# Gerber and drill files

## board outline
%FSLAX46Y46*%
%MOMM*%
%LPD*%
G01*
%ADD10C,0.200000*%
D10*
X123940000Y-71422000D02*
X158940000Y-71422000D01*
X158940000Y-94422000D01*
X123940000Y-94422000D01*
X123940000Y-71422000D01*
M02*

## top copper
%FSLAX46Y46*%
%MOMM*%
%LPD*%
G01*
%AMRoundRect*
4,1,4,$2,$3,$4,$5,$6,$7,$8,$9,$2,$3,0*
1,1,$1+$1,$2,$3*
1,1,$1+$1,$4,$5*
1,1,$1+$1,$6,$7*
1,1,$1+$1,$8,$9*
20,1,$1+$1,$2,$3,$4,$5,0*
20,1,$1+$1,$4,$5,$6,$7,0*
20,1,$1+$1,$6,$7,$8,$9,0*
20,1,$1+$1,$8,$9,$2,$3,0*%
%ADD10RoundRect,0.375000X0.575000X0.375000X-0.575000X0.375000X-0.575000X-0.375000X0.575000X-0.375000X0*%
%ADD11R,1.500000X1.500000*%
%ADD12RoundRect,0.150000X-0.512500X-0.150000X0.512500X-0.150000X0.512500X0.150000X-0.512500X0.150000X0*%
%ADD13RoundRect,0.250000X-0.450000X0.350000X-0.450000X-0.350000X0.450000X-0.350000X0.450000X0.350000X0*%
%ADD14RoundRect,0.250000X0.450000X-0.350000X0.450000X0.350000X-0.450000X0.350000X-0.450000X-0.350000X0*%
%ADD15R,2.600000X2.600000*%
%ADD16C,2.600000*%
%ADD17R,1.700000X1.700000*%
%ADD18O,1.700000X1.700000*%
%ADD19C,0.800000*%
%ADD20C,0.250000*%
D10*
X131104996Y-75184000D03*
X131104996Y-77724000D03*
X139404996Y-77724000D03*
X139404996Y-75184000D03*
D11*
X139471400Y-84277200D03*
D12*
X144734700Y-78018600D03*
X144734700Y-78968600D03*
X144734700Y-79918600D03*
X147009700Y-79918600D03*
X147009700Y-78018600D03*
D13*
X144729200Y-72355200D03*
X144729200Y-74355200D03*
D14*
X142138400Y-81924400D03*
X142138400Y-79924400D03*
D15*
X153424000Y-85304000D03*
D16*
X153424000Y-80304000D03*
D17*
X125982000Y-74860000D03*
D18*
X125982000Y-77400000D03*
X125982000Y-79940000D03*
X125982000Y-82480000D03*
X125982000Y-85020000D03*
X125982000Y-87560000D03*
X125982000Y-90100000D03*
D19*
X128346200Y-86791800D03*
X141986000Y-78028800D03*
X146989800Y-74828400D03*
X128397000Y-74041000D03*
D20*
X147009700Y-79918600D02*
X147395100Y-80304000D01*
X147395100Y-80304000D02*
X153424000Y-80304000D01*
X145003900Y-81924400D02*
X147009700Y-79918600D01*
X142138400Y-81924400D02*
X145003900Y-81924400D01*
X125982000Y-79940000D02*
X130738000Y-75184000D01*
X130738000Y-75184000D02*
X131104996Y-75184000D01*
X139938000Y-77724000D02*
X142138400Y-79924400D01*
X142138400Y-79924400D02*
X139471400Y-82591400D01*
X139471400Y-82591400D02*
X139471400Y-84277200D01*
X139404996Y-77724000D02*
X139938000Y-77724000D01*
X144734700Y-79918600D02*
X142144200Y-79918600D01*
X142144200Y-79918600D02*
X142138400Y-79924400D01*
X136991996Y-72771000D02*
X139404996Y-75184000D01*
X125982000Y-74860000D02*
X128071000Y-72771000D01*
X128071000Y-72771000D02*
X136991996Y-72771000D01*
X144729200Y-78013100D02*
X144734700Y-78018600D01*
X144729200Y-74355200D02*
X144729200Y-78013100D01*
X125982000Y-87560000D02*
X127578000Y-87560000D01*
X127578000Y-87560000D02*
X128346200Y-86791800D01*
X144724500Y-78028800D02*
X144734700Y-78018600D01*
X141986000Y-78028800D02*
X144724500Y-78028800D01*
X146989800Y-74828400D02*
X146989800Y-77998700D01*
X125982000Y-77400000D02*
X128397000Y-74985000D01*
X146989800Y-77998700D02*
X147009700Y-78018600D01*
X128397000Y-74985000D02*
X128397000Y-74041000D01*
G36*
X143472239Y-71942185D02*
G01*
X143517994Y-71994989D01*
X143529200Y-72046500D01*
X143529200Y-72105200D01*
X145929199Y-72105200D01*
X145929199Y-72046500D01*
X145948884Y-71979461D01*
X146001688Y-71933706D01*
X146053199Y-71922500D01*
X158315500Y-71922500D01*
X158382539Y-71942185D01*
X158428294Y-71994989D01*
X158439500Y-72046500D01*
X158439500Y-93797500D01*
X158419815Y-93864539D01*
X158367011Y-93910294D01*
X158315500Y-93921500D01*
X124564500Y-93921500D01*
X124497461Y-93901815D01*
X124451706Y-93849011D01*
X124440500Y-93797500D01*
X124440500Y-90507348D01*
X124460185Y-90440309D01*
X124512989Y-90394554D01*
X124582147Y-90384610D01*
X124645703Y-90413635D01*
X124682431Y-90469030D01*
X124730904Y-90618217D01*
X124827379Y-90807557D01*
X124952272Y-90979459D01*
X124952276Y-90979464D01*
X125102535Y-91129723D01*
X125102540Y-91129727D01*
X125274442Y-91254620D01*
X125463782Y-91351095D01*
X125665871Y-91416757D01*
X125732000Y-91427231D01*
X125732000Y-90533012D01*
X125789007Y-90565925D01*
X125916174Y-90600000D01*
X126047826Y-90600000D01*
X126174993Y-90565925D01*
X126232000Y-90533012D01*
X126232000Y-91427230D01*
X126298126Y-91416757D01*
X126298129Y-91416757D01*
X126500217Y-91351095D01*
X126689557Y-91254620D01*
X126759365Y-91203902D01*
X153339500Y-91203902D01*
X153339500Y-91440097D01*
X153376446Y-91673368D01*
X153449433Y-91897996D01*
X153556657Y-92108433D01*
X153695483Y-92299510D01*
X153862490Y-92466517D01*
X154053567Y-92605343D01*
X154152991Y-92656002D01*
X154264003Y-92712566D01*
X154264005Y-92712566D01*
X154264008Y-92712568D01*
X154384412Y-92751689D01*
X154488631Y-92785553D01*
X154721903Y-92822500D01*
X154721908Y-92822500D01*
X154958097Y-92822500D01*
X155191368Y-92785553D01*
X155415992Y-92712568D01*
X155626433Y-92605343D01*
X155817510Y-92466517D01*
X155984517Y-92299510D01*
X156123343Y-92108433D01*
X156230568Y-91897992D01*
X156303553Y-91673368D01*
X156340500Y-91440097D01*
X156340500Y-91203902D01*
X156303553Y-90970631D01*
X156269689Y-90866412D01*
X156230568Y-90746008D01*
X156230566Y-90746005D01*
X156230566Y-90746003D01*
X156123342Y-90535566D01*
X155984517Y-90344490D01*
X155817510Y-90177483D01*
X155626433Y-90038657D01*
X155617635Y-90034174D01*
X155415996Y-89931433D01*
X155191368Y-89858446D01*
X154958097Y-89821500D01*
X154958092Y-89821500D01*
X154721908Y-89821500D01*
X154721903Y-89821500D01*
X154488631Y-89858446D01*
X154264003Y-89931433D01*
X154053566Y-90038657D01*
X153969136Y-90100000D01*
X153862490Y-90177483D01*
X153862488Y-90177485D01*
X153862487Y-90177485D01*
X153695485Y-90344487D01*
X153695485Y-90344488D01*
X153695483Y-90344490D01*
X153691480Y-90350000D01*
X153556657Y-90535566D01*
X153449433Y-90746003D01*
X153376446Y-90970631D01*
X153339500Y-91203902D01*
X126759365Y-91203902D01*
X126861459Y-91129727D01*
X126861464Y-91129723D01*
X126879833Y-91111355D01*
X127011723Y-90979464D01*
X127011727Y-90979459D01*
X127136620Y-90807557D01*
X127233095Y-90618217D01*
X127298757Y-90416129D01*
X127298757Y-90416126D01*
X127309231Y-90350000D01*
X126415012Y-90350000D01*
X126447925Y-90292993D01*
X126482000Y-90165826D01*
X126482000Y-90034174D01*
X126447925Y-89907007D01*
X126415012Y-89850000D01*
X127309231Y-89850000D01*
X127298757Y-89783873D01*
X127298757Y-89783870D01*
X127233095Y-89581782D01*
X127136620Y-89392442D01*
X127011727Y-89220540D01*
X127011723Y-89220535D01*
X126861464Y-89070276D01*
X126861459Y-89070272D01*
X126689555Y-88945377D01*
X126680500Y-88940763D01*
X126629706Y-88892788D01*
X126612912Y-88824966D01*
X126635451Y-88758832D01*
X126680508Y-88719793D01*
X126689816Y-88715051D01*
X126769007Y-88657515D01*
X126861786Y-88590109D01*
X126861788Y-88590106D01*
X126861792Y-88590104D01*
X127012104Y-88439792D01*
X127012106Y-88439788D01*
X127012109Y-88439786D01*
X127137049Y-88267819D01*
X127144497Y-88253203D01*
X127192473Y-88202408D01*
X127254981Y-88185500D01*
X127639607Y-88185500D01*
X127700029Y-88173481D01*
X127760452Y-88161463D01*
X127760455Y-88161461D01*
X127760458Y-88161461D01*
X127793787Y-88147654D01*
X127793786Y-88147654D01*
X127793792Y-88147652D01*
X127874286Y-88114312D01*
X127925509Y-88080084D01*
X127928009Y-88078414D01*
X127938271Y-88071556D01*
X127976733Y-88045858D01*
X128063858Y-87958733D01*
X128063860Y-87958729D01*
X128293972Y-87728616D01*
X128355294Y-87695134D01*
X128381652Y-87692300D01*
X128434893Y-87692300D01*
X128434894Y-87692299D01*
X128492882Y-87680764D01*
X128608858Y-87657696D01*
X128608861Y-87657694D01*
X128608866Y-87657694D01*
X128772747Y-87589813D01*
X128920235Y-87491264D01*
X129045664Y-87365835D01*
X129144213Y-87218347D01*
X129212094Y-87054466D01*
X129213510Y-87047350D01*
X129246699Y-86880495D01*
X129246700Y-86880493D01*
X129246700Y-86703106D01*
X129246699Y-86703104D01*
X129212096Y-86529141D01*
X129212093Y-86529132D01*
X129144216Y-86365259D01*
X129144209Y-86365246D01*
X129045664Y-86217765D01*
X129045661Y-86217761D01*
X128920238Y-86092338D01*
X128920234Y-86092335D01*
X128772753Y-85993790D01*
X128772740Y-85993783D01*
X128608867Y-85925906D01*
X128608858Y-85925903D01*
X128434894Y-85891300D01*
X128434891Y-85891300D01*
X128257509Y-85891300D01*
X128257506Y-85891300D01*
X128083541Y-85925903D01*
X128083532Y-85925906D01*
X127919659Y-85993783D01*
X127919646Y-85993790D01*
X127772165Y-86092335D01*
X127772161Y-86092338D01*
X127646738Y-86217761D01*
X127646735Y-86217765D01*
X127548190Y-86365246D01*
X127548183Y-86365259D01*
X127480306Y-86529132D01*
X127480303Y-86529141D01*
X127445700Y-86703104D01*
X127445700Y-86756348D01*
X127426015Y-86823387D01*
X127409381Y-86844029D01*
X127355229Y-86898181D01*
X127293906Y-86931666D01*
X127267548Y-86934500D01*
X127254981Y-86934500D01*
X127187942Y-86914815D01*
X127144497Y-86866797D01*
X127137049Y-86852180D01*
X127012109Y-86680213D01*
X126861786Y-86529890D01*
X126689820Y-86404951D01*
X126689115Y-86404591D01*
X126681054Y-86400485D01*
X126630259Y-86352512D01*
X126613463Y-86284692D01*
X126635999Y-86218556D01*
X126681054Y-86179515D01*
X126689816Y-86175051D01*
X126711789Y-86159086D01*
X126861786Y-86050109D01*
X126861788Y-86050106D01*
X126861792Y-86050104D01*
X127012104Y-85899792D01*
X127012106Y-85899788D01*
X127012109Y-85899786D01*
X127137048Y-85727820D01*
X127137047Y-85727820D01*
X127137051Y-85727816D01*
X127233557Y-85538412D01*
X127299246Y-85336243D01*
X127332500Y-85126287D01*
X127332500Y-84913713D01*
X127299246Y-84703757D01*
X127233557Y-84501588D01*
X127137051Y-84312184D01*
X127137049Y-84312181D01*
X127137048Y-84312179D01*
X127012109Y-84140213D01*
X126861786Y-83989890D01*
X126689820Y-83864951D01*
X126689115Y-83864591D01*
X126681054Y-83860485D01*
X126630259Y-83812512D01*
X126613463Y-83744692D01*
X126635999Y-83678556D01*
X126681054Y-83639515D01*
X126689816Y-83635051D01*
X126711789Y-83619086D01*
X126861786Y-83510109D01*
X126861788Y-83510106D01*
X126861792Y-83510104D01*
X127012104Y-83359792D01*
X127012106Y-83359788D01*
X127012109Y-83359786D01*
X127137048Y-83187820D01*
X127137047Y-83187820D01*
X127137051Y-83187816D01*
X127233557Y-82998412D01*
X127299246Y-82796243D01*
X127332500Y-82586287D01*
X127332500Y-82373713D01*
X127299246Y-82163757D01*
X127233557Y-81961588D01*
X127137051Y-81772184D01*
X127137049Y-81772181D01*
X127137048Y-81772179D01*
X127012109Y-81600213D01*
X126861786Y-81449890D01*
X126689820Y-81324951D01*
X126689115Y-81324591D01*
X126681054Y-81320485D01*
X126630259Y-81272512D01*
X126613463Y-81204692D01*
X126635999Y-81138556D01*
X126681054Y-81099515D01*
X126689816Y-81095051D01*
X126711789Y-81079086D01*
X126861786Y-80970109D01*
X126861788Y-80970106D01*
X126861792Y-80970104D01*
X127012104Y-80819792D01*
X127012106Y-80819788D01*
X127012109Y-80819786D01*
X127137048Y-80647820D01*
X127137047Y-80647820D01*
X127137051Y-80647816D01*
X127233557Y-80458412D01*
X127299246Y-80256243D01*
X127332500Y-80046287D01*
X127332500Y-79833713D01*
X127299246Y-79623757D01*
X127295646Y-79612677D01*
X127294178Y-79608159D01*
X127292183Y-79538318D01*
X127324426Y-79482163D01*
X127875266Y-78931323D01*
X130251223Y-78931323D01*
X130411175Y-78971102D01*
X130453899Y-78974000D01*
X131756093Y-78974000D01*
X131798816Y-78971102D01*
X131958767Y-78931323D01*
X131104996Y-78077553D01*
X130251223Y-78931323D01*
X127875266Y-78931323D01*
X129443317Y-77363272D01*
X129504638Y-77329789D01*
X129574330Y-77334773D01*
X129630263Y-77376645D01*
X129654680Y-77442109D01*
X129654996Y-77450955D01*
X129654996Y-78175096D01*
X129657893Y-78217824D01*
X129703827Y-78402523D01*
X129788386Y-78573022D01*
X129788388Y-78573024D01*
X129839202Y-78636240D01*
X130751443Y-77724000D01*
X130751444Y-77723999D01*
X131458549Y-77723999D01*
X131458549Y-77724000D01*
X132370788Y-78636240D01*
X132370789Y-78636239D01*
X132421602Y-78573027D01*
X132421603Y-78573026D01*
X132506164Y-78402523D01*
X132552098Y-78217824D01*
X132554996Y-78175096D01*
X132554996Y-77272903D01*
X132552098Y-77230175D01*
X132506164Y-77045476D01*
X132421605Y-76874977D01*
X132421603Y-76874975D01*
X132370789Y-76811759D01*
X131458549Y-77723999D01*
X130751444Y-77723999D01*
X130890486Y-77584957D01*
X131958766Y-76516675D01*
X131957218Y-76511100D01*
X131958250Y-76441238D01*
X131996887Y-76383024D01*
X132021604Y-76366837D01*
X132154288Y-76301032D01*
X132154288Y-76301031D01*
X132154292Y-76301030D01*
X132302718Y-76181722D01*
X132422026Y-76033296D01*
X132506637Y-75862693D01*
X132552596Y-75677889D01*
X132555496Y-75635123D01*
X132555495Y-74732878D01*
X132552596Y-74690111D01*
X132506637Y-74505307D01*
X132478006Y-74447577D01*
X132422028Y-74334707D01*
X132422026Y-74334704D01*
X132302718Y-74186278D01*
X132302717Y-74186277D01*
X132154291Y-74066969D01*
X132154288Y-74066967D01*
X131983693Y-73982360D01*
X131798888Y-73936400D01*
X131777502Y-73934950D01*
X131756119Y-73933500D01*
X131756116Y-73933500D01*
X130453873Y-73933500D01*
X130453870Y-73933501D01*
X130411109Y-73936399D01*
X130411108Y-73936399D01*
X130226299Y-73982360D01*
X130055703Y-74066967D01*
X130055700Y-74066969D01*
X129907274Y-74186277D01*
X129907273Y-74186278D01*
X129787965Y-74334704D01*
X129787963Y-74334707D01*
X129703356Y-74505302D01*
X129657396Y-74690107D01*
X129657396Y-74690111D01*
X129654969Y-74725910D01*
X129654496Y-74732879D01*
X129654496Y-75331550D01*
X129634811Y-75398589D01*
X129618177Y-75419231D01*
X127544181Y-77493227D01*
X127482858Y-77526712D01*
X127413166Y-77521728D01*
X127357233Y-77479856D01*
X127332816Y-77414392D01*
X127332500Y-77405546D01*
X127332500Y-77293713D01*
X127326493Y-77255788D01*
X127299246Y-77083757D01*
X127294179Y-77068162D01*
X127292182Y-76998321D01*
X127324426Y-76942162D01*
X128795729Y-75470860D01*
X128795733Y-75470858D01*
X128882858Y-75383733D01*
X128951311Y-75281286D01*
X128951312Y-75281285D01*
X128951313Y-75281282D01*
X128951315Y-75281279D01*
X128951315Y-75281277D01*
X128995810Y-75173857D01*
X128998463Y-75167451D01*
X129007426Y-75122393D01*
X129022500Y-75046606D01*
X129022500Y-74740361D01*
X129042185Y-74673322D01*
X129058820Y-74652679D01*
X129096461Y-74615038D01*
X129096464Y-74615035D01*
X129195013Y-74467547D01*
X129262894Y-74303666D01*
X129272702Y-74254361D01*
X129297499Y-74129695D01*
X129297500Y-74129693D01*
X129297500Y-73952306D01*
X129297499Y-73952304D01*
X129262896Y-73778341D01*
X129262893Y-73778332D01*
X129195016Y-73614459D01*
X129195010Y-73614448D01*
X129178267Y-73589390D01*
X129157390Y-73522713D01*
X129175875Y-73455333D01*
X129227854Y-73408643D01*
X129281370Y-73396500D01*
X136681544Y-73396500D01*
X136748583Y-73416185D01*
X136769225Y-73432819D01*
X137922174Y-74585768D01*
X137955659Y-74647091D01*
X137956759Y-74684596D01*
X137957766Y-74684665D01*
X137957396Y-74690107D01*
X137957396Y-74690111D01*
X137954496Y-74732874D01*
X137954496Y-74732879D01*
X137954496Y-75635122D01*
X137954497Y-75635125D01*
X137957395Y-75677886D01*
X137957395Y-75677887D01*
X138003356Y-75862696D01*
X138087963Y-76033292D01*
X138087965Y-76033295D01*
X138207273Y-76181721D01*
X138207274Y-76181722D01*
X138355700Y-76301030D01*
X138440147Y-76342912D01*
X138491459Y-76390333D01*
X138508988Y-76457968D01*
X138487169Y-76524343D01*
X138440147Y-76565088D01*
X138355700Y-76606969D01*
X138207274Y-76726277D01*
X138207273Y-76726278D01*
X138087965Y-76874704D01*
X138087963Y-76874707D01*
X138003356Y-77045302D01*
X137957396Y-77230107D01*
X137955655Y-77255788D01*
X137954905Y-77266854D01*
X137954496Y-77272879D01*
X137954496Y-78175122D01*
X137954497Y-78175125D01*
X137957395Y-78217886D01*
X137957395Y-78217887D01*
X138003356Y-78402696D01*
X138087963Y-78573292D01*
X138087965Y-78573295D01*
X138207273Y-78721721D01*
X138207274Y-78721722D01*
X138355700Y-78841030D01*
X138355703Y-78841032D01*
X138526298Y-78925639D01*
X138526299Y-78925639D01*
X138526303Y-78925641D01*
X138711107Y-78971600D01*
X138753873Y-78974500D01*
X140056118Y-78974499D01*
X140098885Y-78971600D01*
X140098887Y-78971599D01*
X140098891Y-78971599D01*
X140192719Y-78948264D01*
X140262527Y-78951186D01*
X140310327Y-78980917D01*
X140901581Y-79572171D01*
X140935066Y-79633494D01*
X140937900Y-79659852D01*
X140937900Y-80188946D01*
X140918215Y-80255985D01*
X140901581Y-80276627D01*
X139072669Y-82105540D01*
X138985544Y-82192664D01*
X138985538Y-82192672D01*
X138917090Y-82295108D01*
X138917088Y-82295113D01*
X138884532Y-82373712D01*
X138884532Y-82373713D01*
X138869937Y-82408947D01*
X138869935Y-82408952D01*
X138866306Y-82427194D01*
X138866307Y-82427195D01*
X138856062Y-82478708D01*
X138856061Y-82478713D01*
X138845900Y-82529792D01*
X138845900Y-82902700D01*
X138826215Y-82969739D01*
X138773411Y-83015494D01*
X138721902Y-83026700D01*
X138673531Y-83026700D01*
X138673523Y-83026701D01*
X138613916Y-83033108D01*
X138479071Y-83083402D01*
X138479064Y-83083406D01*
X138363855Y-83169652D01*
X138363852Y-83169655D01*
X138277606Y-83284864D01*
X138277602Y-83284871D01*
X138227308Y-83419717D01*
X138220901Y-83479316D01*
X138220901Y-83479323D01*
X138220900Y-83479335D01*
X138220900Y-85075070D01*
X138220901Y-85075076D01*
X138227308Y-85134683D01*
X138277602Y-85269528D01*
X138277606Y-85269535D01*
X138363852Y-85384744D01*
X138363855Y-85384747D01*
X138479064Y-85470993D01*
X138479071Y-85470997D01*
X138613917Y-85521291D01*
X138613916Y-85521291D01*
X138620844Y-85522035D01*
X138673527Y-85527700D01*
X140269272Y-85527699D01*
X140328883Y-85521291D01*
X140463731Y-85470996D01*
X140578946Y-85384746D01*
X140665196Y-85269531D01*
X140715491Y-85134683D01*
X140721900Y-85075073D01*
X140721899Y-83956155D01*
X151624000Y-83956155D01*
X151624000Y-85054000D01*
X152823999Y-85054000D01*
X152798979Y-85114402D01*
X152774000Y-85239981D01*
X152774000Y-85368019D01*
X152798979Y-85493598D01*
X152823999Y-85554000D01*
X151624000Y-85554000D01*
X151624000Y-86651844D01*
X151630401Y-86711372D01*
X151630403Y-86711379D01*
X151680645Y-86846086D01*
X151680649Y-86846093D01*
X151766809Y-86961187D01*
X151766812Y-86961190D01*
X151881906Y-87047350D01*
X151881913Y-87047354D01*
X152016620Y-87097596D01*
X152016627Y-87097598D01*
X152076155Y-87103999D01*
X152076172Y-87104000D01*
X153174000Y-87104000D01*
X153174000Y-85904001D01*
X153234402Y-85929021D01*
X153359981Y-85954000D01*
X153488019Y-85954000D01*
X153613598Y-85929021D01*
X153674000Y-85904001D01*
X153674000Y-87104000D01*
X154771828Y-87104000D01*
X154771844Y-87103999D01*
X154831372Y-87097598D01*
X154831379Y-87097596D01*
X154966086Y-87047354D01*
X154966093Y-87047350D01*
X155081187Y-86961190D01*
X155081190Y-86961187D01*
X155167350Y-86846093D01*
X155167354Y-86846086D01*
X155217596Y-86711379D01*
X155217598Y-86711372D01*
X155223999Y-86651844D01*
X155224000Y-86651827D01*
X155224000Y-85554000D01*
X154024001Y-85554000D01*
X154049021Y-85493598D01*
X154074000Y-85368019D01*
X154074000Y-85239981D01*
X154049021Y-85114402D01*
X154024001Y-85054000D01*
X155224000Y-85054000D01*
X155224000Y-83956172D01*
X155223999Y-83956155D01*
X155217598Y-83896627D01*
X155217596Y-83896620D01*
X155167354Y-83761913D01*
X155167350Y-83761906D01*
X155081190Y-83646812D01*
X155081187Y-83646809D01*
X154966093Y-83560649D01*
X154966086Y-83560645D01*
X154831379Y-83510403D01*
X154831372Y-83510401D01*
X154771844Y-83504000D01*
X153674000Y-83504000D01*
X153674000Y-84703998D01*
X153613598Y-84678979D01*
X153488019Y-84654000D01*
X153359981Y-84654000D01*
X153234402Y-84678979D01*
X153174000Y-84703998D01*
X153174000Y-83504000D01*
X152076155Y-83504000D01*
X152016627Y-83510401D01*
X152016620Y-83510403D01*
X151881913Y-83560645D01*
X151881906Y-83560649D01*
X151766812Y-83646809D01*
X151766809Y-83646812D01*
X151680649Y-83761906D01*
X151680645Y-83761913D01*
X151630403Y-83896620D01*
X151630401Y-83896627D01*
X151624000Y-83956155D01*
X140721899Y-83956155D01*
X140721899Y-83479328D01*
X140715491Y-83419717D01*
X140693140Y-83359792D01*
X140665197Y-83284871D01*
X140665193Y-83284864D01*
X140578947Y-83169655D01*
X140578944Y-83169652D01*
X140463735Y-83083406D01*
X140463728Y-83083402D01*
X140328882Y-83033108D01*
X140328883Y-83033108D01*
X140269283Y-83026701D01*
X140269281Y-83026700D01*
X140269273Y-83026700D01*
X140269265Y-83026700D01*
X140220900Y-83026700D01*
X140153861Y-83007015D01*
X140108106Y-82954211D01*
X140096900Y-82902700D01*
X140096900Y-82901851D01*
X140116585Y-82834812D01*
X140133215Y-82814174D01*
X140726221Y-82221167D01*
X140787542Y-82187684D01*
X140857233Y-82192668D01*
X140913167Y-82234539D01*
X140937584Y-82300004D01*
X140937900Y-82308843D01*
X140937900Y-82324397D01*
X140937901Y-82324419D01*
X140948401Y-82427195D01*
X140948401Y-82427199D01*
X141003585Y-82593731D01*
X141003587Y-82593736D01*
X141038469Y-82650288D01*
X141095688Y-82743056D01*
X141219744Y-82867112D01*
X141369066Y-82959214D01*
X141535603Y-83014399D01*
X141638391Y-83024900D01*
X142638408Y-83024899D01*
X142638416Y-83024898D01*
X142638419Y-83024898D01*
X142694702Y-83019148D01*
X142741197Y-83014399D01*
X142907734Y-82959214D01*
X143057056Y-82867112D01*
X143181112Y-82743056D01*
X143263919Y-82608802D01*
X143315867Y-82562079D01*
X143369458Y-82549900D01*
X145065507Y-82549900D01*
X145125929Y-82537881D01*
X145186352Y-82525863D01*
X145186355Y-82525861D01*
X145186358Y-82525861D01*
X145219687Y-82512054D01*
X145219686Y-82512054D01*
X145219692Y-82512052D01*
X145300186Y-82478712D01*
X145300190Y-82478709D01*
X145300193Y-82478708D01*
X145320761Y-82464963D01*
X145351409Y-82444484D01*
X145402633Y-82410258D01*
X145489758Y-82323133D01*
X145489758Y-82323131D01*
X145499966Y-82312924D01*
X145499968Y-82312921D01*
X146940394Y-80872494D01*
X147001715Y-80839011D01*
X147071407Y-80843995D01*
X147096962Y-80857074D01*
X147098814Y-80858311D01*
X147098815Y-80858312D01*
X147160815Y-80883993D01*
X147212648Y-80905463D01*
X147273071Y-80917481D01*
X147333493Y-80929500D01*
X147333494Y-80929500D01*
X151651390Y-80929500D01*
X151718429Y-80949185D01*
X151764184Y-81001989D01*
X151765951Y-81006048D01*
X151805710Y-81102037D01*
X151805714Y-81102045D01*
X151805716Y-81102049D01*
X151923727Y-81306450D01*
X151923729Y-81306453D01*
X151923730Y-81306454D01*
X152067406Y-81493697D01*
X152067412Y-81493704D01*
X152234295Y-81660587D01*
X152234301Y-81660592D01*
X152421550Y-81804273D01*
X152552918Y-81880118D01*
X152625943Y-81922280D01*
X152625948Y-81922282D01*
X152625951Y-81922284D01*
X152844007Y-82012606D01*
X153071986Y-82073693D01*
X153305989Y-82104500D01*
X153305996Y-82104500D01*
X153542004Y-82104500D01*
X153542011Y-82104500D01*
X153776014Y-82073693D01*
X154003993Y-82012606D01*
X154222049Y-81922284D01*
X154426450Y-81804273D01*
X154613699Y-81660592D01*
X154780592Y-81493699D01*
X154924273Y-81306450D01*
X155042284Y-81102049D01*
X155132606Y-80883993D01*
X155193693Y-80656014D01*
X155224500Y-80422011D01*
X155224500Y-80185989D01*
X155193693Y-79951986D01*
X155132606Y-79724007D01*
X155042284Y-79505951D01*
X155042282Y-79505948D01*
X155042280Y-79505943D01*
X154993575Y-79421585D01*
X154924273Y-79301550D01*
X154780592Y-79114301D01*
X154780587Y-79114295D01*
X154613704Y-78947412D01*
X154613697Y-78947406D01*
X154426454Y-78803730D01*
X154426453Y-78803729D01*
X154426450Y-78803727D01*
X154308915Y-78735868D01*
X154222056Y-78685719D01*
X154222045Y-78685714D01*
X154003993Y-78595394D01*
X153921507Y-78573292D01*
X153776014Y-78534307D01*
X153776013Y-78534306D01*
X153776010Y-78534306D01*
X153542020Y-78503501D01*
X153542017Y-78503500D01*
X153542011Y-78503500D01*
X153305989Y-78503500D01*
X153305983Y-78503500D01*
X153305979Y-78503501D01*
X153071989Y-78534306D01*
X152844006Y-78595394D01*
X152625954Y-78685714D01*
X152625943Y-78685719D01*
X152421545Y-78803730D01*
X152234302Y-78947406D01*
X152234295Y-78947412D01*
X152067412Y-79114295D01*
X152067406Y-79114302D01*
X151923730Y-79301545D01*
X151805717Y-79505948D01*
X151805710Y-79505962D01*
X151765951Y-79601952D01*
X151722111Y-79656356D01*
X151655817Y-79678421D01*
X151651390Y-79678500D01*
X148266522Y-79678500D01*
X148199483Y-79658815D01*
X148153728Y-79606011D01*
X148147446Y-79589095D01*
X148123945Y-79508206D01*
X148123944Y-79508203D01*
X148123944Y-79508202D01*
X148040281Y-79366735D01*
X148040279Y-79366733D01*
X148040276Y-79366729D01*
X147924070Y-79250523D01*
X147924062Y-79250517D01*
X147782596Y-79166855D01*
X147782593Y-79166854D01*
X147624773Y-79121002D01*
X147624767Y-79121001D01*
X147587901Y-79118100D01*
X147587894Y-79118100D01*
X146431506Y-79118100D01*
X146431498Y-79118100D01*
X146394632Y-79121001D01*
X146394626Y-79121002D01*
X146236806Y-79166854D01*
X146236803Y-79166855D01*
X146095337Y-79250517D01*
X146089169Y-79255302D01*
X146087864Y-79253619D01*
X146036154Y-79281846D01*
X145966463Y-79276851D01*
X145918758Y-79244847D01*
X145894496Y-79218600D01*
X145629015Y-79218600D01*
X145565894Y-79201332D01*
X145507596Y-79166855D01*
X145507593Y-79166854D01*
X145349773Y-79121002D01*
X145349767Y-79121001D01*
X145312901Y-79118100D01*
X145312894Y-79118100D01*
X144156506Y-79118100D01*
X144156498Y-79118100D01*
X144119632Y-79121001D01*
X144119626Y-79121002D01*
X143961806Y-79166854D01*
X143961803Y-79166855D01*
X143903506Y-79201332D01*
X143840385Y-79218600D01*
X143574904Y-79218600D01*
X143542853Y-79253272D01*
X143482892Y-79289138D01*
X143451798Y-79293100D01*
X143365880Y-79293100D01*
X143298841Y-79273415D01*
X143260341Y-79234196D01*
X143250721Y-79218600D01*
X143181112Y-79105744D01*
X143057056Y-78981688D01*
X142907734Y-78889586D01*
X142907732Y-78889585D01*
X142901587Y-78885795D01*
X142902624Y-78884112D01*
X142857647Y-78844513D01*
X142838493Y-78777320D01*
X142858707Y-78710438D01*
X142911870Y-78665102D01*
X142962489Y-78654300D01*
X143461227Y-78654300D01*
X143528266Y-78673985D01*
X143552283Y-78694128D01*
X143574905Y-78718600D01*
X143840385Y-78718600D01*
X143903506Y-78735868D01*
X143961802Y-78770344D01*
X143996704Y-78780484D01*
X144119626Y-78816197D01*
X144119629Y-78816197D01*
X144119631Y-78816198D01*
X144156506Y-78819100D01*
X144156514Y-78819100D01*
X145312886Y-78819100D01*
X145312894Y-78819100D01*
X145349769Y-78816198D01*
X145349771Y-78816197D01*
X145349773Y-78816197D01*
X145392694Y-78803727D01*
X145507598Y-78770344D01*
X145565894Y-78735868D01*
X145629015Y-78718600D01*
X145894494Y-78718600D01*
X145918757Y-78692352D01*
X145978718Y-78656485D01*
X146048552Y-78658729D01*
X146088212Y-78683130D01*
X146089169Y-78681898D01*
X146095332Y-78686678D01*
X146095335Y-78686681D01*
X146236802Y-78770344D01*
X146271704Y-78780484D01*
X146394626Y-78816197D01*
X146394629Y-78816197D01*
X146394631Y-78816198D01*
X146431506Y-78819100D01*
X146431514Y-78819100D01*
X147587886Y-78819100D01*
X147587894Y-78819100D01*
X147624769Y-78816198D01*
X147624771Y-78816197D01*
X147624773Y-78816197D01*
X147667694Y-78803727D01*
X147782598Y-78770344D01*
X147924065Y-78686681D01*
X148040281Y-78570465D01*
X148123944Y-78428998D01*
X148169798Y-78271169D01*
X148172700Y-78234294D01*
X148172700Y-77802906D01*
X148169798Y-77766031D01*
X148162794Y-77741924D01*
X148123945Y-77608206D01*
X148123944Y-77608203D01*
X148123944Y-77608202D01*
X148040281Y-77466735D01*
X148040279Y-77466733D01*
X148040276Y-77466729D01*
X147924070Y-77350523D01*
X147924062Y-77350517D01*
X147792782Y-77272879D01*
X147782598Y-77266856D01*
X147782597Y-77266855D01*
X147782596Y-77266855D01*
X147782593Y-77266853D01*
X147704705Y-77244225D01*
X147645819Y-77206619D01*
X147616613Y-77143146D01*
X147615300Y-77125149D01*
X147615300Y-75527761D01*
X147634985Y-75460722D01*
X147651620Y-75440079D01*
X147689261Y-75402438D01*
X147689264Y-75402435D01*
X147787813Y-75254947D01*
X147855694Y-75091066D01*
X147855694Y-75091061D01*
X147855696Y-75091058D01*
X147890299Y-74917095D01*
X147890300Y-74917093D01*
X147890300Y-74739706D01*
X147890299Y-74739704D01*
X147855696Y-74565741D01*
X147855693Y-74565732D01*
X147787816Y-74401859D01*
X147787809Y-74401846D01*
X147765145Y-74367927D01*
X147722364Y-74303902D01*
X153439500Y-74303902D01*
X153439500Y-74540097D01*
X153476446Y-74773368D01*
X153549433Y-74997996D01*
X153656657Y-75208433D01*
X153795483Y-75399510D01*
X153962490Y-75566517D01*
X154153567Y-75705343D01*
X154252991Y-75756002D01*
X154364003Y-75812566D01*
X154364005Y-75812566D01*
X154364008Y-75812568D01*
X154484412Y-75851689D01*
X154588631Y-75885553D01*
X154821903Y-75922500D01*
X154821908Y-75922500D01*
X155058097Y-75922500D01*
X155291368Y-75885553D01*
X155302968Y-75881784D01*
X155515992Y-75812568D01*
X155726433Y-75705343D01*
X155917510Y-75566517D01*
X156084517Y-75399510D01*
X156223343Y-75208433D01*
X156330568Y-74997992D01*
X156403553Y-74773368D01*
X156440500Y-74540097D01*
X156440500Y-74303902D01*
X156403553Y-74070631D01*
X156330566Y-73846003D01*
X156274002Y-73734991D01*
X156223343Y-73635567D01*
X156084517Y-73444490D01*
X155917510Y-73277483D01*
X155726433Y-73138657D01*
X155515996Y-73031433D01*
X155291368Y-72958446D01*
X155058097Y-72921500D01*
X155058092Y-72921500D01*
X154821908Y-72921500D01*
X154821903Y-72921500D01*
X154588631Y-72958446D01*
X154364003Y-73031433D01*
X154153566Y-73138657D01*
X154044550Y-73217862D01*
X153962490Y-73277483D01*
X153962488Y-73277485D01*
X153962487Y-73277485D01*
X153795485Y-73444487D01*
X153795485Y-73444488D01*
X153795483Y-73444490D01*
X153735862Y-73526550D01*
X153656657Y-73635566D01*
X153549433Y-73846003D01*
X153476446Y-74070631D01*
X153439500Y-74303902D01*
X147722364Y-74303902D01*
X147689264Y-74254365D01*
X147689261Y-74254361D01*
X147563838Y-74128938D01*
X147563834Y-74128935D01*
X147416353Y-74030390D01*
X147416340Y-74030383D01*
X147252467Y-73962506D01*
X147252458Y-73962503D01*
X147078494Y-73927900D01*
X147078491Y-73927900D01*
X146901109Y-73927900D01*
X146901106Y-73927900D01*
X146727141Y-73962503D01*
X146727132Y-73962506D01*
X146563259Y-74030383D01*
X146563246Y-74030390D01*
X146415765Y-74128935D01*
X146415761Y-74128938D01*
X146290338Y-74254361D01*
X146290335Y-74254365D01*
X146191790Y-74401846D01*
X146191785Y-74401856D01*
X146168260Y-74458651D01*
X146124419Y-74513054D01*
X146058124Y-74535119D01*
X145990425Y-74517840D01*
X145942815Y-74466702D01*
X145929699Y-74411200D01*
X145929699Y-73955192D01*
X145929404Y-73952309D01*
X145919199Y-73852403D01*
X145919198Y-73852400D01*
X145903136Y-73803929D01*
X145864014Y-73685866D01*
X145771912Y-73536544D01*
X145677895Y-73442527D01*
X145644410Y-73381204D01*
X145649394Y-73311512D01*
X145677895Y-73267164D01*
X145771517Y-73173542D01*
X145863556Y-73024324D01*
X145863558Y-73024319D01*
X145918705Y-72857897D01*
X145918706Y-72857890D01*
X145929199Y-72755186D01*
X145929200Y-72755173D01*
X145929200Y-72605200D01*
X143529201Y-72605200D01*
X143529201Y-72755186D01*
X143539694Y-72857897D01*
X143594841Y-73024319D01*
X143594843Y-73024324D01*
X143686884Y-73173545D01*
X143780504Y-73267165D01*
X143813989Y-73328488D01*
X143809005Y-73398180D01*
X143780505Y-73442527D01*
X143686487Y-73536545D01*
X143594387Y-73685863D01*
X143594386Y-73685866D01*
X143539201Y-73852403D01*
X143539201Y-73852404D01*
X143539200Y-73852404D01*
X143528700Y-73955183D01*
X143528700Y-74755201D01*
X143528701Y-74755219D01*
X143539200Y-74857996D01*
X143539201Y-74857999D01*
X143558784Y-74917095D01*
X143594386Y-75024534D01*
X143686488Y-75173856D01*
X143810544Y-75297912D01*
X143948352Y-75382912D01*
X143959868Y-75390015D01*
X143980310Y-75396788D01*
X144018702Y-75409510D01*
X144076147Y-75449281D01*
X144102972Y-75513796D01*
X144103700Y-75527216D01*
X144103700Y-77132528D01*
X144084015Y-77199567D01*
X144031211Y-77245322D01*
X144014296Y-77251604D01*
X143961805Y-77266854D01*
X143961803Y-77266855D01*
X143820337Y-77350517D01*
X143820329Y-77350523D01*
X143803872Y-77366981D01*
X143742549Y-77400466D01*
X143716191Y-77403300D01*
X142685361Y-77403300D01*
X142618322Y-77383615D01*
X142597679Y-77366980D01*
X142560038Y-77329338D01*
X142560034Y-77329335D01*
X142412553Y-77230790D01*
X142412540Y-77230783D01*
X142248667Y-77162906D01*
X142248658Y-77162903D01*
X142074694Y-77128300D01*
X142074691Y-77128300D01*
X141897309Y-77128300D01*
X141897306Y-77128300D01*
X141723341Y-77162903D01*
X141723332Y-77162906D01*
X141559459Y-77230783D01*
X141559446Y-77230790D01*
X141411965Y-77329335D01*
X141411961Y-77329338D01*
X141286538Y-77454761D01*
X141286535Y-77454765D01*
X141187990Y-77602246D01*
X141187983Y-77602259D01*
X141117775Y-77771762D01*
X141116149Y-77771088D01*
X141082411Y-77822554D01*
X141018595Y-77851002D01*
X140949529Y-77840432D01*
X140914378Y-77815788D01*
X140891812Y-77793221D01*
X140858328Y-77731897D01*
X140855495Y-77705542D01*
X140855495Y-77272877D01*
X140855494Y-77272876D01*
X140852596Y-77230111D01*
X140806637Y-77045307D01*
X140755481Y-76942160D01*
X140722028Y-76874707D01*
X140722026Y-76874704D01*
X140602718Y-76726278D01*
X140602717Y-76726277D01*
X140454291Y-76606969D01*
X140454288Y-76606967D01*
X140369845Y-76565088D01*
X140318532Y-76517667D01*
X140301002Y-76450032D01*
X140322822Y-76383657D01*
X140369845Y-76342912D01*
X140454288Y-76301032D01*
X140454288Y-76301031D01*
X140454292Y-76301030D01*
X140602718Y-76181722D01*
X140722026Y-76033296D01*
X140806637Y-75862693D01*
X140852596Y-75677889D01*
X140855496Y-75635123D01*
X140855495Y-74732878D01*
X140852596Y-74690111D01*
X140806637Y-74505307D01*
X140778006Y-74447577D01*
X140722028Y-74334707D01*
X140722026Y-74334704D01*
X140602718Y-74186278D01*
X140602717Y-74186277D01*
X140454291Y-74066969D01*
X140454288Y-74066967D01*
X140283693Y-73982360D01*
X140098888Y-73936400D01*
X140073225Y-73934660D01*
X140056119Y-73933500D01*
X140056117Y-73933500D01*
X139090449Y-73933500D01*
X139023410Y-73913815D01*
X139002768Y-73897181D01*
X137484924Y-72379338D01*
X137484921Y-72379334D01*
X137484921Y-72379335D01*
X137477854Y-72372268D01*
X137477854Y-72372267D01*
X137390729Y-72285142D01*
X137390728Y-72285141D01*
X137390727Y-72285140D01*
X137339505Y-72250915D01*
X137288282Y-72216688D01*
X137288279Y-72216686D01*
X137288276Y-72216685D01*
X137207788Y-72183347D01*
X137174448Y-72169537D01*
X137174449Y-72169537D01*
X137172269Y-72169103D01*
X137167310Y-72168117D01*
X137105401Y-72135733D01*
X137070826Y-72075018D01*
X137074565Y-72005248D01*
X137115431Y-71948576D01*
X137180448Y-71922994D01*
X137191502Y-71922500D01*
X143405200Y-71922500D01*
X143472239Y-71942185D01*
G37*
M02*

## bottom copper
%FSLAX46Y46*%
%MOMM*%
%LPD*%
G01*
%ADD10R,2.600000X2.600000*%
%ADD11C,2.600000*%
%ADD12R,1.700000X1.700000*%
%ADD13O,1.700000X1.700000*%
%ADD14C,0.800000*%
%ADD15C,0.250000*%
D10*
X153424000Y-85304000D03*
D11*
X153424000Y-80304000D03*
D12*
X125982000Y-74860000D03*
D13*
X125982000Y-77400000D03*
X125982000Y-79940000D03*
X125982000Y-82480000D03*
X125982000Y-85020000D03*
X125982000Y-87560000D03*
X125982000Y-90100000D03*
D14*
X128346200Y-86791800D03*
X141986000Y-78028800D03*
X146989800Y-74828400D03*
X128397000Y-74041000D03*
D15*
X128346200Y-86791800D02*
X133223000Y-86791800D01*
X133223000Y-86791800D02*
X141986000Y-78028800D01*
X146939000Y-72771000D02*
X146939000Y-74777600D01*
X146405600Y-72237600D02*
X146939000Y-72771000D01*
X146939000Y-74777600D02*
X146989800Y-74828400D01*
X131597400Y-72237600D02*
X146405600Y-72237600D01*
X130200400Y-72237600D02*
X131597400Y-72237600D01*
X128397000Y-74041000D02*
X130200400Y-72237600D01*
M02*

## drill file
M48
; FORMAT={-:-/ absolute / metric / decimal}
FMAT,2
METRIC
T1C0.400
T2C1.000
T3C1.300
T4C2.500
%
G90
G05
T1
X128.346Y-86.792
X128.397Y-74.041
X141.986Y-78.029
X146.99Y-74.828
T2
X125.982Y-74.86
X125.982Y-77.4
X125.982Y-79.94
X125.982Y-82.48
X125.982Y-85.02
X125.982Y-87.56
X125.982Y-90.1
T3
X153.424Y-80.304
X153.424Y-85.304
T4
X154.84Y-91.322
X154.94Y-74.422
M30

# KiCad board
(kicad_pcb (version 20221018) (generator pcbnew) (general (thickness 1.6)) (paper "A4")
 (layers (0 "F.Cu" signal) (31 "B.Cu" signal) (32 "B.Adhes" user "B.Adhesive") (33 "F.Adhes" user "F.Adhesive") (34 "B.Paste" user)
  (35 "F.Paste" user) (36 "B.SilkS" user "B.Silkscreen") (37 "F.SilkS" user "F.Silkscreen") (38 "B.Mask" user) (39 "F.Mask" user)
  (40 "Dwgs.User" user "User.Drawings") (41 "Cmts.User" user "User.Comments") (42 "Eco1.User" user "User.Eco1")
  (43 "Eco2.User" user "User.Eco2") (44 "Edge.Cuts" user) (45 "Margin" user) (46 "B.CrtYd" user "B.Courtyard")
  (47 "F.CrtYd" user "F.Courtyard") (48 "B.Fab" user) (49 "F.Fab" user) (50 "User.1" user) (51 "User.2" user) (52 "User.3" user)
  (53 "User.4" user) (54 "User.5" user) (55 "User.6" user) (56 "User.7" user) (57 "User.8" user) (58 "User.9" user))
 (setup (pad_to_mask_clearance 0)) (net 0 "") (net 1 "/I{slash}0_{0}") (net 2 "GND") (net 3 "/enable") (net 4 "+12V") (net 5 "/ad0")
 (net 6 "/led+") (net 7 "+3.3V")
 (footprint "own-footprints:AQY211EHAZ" (layer "F.Cu") (at 135.255 76.454 90)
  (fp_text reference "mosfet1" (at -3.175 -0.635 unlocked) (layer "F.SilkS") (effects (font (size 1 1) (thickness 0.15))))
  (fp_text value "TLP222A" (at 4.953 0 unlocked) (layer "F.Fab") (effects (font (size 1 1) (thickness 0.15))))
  (pad "1" smd roundrect (at 1.27 -4.150004 180) (size 1.9 1.5) (layers "F.Cu" "F.Paste" "F.Mask") (roundrect_rratio 0.25)
   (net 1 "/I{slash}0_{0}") (thermal_bridge_angle 45))
  (pad "2" smd roundrect (at -1.27 -4.150004 180) (size 1.9 1.5) (layers "F.Cu" "F.Paste" "F.Mask") (roundrect_rratio 0.25) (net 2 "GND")
   (thermal_bridge_angle 45))
  (pad "3" smd roundrect (at -1.27 4.149996 180) (size 1.9 1.5) (layers "F.Cu" "F.Paste" "F.Mask") (roundrect_rratio 0.25) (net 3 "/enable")
   (thermal_bridge_angle 45))
  (pad "4" smd roundrect (at 1.27 4.149996 180) (size 1.9 1.5) (layers "F.Cu" "F.Paste" "F.Mask") (roundrect_rratio 0.25) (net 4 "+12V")
   (thermal_bridge_angle 45)))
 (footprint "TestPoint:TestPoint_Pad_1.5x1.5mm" (layer "F.Cu") (at 139.4714 84.2772)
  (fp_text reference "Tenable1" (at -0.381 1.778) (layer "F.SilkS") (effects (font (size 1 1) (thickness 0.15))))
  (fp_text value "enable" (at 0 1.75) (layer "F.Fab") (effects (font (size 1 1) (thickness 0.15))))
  (pad "1" smd rect (at 0 0) (size 1.5 1.5) (layers "F.Cu" "F.Mask") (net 3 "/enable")))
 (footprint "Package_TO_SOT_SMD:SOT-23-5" (layer "F.Cu") (at 145.8722 78.9686)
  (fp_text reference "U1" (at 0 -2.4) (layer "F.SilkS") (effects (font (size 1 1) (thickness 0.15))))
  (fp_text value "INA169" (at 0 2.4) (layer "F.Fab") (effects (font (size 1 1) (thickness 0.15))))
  (pad "1" smd roundrect (at -1.1375 -0.95) (size 1.325 0.6) (layers "F.Cu" "F.Paste" "F.Mask") (roundrect_rratio 0.25) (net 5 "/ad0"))
  (pad "2" smd roundrect (at -1.1375 0) (size 1.325 0.6) (layers "F.Cu" "F.Paste" "F.Mask") (roundrect_rratio 0.25) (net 2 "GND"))
  (pad "3" smd roundrect (at -1.1375 0.95) (size 1.325 0.6) (layers "F.Cu" "F.Paste" "F.Mask") (roundrect_rratio 0.25) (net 3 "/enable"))
  (pad "4" smd roundrect (at 1.1375 0.95) (size 1.325 0.6) (layers "F.Cu" "F.Paste" "F.Mask") (roundrect_rratio 0.25) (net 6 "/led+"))
  (pad "5" smd roundrect (at 1.1375 -0.95) (size 1.325 0.6) (layers "F.Cu" "F.Paste" "F.Mask") (roundrect_rratio 0.25) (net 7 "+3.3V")))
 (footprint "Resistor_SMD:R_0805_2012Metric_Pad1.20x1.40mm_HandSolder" (layer "F.Cu") (at 144.7292 73.3552 -90)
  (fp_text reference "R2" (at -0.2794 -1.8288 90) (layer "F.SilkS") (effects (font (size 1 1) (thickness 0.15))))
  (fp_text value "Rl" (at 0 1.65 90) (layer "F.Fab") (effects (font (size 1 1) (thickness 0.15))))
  (pad "1" smd roundrect (at -1 0 270) (size 1.2 1.4) (layers "F.Cu" "F.Paste" "F.Mask") (roundrect_rratio 0.208333) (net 2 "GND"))
  (pad "2" smd roundrect (at 1 0 270) (size 1.2 1.4) (layers "F.Cu" "F.Paste" "F.Mask") (roundrect_rratio 0.208333) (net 5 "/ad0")))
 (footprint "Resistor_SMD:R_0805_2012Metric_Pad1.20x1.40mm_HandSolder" (layer "F.Cu") (at 142.1384 80.9244 90)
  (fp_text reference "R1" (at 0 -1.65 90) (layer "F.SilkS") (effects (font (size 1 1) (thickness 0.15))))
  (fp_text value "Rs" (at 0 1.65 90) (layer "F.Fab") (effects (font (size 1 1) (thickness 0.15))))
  (pad "1" smd roundrect (at -1 0 90) (size 1.2 1.4) (layers "F.Cu" "F.Paste" "F.Mask") (roundrect_rratio 0.208333) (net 6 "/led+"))
  (pad "2" smd roundrect (at 1 0 90) (size 1.2 1.4) (layers "F.Cu" "F.Paste" "F.Mask") (roundrect_rratio 0.208333) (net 3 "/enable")))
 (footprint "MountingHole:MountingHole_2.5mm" (layer "F.Cu") (at 154.84 91.322)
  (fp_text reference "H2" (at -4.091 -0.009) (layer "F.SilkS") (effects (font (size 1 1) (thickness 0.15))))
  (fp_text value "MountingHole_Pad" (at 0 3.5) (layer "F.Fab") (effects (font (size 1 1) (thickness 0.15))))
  (pad "" np_thru_hole circle (at 0 0) (size 2.5 2.5) (drill 2.5) (layers "*.Cu" "*.Mask")))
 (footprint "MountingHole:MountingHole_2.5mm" (layer "F.Cu") (at 154.94 74.422)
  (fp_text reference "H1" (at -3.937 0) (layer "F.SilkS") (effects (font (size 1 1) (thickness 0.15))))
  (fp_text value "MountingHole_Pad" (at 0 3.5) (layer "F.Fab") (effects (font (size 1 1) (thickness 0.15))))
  (pad "" np_thru_hole circle (at 0 0) (size 2.5 2.5) (drill 2.5) (layers "*.Cu" "*.Mask")))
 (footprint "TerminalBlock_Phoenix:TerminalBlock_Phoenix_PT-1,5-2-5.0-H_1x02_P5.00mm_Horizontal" (layer "F.Cu") (at 153.424 85.304 90)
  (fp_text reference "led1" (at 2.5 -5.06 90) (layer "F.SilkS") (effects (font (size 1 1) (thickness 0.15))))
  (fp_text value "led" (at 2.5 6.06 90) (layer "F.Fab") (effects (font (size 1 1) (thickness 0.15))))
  (pad "1" thru_hole rect (at 0 0 90) (size 2.6 2.6) (drill 1.3) (layers "*.Cu" "*.Mask") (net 2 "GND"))
  (pad "2" thru_hole circle (at 5 0 90) (size 2.6 2.6) (drill 1.3) (layers "*.Cu" "*.Mask") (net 6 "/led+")))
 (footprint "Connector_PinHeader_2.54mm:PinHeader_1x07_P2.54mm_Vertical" (layer "B.Cu") (at 125.982 74.86 180)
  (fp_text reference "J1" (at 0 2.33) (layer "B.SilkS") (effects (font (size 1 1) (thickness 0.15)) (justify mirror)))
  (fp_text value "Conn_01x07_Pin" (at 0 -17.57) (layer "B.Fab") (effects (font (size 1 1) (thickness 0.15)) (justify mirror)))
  (pad "1" thru_hole rect (at 0 0 180) (size 1.7 1.7) (drill 1) (layers "*.Cu" "*.Mask") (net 4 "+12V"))
  (pad "2" thru_hole oval (at 0 -2.54 180) (size 1.7 1.7) (drill 1) (layers "*.Cu" "*.Mask") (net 7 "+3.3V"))
  (pad "3" thru_hole oval (at 0 -5.08 180) (size 1.7 1.7) (drill 1) (layers "*.Cu" "*.Mask") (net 1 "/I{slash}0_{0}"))
  (pad "4" thru_hole oval (at 0 -7.62 180) (size 1.7 1.7) (drill 1) (layers "*.Cu" "*.Mask"))
  (pad "5" thru_hole oval (at 0 -10.16 180) (size 1.7 1.7) (drill 1) (layers "*.Cu" "*.Mask"))
  (pad "6" thru_hole oval (at 0 -12.7 180) (size 1.7 1.7) (drill 1) (layers "*.Cu" "*.Mask") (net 5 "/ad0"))
  (pad "7" thru_hole oval (at 0 -15.24 180) (size 1.7 1.7) (drill 1) (layers "*.Cu" "*.Mask") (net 2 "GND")))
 (gr_rect (start 123.94 71.422) (end 158.94 94.422) (stroke (width 0.2) (type default)) (fill none) (layer "Edge.Cuts"))
 (segment (start 147.0097 79.9186) (end 147.3951 80.304) (width 0.25) (layer "F.Cu") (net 6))
 (segment (start 147.3951 80.304) (end 153.424 80.304) (width 0.25) (layer "F.Cu") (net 6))
 (segment (start 145.0039 81.9244) (end 147.0097 79.9186) (width 0.25) (layer "F.Cu") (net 6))
 (segment (start 142.1384 81.9244) (end 145.0039 81.9244) (width 0.25) (layer "F.Cu") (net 6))
 (segment (start 125.982 79.94) (end 130.738 75.184) (width 0.25) (layer "F.Cu") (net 1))
 (segment (start 130.738 75.184) (end 131.104996 75.184) (width 0.25) (layer "F.Cu") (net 1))
 (segment (start 139.938 77.724) (end 142.1384 79.9244) (width 0.25) (layer "F.Cu") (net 3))
 (segment (start 142.1384 79.9244) (end 139.4714 82.5914) (width 0.25) (layer "F.Cu") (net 3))
 (segment (start 139.4714 82.5914) (end 139.4714 84.2772) (width 0.25) (layer "F.Cu") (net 3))
 (segment (start 139.404996 77.724) (end 139.938 77.724) (width 0.25) (layer "F.Cu") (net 3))
 (segment (start 144.7347 79.9186) (end 142.1442 79.9186) (width 0.25) (layer "F.Cu") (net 3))
 (segment (start 142.1442 79.9186) (end 142.1384 79.9244) (width 0.25) (layer "F.Cu") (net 3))
 (segment (start 136.991996 72.771) (end 139.404996 75.184) (width 0.25) (layer "F.Cu") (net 4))
 (segment (start 125.982 74.86) (end 128.071 72.771) (width 0.25) (layer "F.Cu") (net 4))
 (segment (start 128.071 72.771) (end 136.991996 72.771) (width 0.25) (layer "F.Cu") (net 4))
 (segment (start 144.7292 78.0131) (end 144.7347 78.0186) (width 0.25) (layer "F.Cu") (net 5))
 (segment (start 144.7292 74.3552) (end 144.7292 78.0131) (width 0.25) (layer "F.Cu") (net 5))
 (segment (start 125.982 87.56) (end 127.578 87.56) (width 0.25) (layer "F.Cu") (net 5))
 (segment (start 127.578 87.56) (end 128.3462 86.7918) (width 0.25) (layer "F.Cu") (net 5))
 (segment (start 144.7245 78.0288) (end 144.7347 78.0186) (width 0.25) (layer "F.Cu") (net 5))
 (segment (start 141.986 78.0288) (end 144.7245 78.0288) (width 0.25) (layer "F.Cu") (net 5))
 (via (at 128.3462 86.7918) (size 0.8) (drill 0.4) (layers "F.Cu" "B.Cu") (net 5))
 (via (at 141.986 78.0288) (size 0.8) (drill 0.4) (layers "F.Cu" "B.Cu") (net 5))
 (segment (start 128.3462 86.7918) (end 133.223 86.7918) (width 0.25) (layer "B.Cu") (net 5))
 (segment (start 133.223 86.7918) (end 141.986 78.0288) (width 0.25) (layer "B.Cu") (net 5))
 (segment (start 146.9898 74.8284) (end 146.9898 77.9987) (width 0.25) (layer "F.Cu") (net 7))
 (segment (start 125.982 77.4) (end 128.397 74.985) (width 0.25) (layer "F.Cu") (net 7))
 (segment (start 146.9898 77.9987) (end 147.0097 78.0186) (width 0.25) (layer "F.Cu") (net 7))
 (segment (start 128.397 74.985) (end 128.397 74.041) (width 0.25) (layer "F.Cu") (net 7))
 (via (at 146.9898 74.8284) (size 0.8) (drill 0.4) (layers "F.Cu" "B.Cu") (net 7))
 (via (at 128.397 74.041) (size 0.8) (drill 0.4) (layers "F.Cu" "B.Cu") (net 7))
 (segment (start 146.939 72.771) (end 146.939 74.7776) (width 0.25) (layer "B.Cu") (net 7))
 (segment (start 146.4056 72.2376) (end 146.939 72.771) (width 0.25) (layer "B.Cu") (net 7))
 (segment (start 146.939 74.7776) (end 146.9898 74.8284) (width 0.25) (layer "B.Cu") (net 7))
 (segment (start 131.5974 72.2376) (end 146.4056 72.2376) (width 0.25) (layer "B.Cu") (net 7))
 (segment (start 130.2004 72.2376) (end 131.5974 72.2376) (width 0.25) (layer "B.Cu") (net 7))
 (segment (start 128.397 74.041) (end 130.2004 72.2376) (width 0.25) (layer "B.Cu") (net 7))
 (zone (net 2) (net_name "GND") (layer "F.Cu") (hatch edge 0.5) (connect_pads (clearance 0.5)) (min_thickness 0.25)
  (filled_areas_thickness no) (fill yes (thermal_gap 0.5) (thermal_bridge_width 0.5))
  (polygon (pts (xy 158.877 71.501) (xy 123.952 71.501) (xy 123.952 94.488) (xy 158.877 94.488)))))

